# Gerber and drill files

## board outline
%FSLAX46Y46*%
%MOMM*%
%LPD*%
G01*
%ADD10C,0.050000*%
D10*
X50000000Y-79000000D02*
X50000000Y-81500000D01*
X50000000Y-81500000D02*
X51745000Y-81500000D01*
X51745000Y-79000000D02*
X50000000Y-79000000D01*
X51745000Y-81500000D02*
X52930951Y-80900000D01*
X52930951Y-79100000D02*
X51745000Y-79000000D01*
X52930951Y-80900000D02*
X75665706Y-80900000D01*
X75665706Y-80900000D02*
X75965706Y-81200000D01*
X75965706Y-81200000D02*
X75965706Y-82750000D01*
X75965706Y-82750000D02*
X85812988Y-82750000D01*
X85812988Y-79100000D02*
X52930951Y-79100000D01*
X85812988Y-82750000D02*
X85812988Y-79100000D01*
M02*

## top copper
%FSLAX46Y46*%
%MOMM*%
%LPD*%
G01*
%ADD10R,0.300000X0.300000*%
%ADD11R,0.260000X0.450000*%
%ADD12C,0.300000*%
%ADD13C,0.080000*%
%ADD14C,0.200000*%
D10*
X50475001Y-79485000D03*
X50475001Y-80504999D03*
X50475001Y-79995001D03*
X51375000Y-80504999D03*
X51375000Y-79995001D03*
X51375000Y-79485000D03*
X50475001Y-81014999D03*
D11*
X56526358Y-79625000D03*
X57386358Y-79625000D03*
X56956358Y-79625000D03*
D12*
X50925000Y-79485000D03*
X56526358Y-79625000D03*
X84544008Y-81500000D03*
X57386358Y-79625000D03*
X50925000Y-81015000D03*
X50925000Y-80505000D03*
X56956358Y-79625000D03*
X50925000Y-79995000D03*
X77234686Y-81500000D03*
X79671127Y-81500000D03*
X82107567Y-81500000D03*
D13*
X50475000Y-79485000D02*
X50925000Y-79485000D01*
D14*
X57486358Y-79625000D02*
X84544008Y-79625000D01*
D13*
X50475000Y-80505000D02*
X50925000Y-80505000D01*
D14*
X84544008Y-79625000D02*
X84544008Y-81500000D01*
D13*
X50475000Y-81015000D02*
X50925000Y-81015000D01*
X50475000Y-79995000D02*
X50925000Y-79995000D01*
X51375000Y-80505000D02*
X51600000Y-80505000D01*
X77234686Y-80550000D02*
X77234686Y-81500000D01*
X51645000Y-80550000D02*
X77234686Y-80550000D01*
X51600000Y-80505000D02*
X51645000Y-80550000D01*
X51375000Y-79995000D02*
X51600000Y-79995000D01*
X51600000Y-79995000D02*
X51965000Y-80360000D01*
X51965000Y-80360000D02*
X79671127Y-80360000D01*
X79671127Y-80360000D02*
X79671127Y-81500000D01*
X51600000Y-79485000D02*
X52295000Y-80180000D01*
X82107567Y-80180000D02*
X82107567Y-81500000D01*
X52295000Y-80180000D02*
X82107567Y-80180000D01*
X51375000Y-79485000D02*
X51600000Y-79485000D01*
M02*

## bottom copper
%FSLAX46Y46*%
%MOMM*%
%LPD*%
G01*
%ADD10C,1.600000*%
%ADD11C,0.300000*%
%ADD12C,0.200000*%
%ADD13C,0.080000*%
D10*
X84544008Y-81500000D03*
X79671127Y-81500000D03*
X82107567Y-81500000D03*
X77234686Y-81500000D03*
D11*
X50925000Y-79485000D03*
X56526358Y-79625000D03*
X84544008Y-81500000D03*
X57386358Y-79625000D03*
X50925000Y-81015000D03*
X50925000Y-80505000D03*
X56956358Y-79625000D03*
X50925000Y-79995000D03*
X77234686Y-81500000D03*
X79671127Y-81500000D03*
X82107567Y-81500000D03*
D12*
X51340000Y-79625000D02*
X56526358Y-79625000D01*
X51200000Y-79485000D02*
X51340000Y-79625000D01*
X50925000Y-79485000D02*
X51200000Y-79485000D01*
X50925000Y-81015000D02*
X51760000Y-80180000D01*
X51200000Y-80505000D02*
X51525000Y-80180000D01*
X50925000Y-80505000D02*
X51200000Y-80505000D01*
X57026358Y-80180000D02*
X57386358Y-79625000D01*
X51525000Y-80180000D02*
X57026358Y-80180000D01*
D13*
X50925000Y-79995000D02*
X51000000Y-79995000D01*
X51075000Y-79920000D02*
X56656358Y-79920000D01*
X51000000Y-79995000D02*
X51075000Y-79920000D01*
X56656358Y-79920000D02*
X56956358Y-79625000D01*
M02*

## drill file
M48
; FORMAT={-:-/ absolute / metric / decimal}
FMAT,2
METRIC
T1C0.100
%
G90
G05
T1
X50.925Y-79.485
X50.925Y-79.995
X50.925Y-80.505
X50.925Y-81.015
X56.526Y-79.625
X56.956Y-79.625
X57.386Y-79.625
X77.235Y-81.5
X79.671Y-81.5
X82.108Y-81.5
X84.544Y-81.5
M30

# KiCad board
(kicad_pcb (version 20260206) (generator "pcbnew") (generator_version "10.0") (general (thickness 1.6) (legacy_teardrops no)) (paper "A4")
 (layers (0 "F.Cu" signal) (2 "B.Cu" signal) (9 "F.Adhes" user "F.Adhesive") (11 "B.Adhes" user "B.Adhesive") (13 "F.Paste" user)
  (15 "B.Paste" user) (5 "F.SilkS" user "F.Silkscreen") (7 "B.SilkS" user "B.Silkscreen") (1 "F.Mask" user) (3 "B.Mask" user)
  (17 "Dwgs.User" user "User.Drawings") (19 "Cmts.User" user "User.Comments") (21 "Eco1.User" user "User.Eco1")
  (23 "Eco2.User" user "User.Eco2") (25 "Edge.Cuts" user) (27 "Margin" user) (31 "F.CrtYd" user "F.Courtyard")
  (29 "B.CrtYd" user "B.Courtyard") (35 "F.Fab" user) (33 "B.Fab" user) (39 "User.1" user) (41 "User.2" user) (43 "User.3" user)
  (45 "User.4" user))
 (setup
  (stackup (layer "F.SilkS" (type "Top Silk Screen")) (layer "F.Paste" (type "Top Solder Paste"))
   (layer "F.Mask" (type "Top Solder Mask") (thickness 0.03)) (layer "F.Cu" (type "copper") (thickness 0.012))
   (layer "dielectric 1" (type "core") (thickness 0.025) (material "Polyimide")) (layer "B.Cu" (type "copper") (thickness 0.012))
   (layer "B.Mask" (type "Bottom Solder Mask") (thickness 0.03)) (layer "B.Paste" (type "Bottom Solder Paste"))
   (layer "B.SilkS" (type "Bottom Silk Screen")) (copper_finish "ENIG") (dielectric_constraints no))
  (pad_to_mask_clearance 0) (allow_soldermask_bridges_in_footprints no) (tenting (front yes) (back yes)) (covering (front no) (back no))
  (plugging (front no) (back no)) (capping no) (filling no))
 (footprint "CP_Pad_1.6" (layer "F.Cu") (at 84.544008 81.5)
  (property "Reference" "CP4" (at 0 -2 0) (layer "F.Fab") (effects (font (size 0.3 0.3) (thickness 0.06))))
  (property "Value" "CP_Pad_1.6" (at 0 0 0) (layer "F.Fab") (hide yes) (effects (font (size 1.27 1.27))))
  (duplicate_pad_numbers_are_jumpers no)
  (pad "1" smd circle (at 0 0) (size 1.6 1.6) (layers "B.Cu" "B.Mask") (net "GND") (solder_mask_margin 0.1)))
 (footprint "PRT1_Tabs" (layer "F.Cu") (at 56.956358 79.625)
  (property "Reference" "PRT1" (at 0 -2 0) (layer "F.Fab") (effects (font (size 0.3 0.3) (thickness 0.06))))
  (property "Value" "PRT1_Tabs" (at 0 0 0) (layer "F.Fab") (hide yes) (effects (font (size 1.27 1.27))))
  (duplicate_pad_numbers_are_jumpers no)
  (pad "1" smd rect (at -0.43 0) (size 0.26 0.45) (layers "F.Cu" "F.Mask") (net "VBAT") (solder_mask_margin 0.05) (thermal_bridge_angle 45))
  (pad "2" smd rect (at 0.43 0) (size 0.26 0.45) (layers "F.Cu" "F.Mask") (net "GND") (solder_mask_margin 0.05) (thermal_bridge_angle 45))
  (pad "3" smd rect (at 0 0) (size 0.26 0.45) (layers "F.Cu" "F.Mask") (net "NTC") (solder_mask_margin 0.05) (thermal_bridge_angle 45)))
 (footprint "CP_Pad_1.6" (layer "F.Cu") (at 77.234686 81.5)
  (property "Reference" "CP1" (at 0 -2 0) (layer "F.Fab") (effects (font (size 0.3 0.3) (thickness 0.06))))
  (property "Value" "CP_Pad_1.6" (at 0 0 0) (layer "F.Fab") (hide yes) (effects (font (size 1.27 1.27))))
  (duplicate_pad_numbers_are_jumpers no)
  (pad "1" smd circle (at 0 0) (size 1.6 1.6) (layers "B.Cu" "B.Mask") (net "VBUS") (solder_mask_margin 0.1)))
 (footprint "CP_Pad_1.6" (layer "F.Cu") (at 79.671127 81.5)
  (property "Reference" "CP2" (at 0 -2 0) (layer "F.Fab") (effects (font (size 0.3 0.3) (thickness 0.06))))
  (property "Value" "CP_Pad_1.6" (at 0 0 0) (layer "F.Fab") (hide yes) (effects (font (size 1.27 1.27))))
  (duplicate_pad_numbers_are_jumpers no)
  (pad "1" smd circle (at 0 0) (size 1.6 1.6) (layers "B.Cu" "B.Mask") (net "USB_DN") (solder_mask_margin 0.1)))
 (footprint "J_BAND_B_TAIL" (layer "F.Cu") (at 50.9 80.25)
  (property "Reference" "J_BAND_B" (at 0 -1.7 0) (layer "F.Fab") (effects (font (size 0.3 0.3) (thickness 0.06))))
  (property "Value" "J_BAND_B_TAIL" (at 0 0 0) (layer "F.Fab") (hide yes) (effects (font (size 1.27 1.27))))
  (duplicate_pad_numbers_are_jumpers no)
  (pad "1" smd rect (at -0.424999 -0.765) (size 0.3 0.3) (layers "F.Cu" "F.Mask") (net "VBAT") (solder_mask_margin 0.05)
   (thermal_bridge_angle 45))
  (pad "2" smd rect (at -0.424999 0.254999) (size 0.3 0.3) (layers "F.Cu" "F.Mask") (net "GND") (solder_mask_margin 0.05)
   (thermal_bridge_angle 45))
  (pad "3" smd rect (at -0.424999 -0.254999) (size 0.3 0.3) (layers "F.Cu" "F.Mask") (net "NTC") (solder_mask_margin 0.05)
   (thermal_bridge_angle 45))
  (pad "4" smd rect (at 0.475 0.254999) (size 0.3 0.3) (layers "F.Cu" "F.Mask") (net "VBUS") (solder_mask_margin 0.05)
   (thermal_bridge_angle 45))
  (pad "5" smd rect (at 0.475 -0.254999) (size 0.3 0.3) (layers "F.Cu" "F.Mask") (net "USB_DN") (solder_mask_margin 0.05)
   (thermal_bridge_angle 45))
  (pad "6" smd rect (at 0.475 -0.765) (size 0.3 0.3) (layers "F.Cu" "F.Mask") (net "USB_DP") (solder_mask_margin 0.05)
   (thermal_bridge_angle 45))
  (pad "7" smd rect (at -0.424999 0.764999) (size 0.3 0.3) (layers "F.Cu" "F.Mask") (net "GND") (solder_mask_margin 0.05)
   (thermal_bridge_angle 45)))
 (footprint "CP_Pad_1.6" (layer "F.Cu") (at 82.107567 81.5)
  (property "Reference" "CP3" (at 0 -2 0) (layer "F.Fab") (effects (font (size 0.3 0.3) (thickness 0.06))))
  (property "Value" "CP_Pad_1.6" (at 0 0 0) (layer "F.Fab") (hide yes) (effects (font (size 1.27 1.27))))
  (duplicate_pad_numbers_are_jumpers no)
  (pad "1" smd circle (at 0 0) (size 1.6 1.6) (layers "B.Cu" "B.Mask") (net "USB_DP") (solder_mask_margin 0.1)))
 (gr_line (start 50 79) (end 50 81.5) (stroke (width 0.05) (type default)) (layer "Edge.Cuts"))
 (gr_line (start 50 81.5) (end 51.745 81.5) (stroke (width 0.05) (type default)) (layer "Edge.Cuts"))
 (gr_line (start 51.745 79) (end 50 79) (stroke (width 0.05) (type default)) (layer "Edge.Cuts"))
 (gr_line (start 51.745 81.5) (end 52.930951 80.9) (stroke (width 0.05) (type default)) (layer "Edge.Cuts"))
 (gr_line (start 52.930951 79.1) (end 51.745 79) (stroke (width 0.05) (type default)) (layer "Edge.Cuts"))
 (gr_line (start 52.930951 80.9) (end 75.665706 80.9) (stroke (width 0.05) (type default)) (layer "Edge.Cuts"))
 (gr_line (start 75.665706 80.9) (end 75.965706 81.2) (stroke (width 0.05) (type default)) (layer "Edge.Cuts"))
 (gr_line (start 75.965706 81.2) (end 75.965706 82.75) (stroke (width 0.05) (type default)) (layer "Edge.Cuts"))
 (gr_line (start 75.965706 82.75) (end 85.812988 82.75) (stroke (width 0.05) (type default)) (layer "Edge.Cuts"))
 (gr_line (start 85.812988 79.1) (end 52.930951 79.1) (stroke (width 0.05) (type default)) (layer "Edge.Cuts"))
 (gr_line (start 85.812988 82.75) (end 85.812988 79.1) (stroke (width 0.05) (type default)) (layer "Edge.Cuts"))
 (segment (start 50.475 79.485) (end 50.925 79.485) (width 0.08) (layer "F.Cu") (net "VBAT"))
 (via (at 56.526358 79.625) (size 0.3) (drill 0.1) (layers "F.Cu" "B.Cu") (tenting (front yes) (back yes)) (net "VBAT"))
 (via (at 50.925 79.485) (size 0.3) (drill 0.1) (layers "F.Cu" "B.Cu") (tenting (front yes) (back yes)) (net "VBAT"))
 (segment (start 50.925 79.485) (end 51.2 79.485) (width 0.2) (layer "B.Cu") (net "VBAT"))
 (segment (start 51.2 79.485) (end 51.34 79.625) (width 0.2) (layer "B.Cu") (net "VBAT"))
 (segment (start 51.34 79.625) (end 56.526358 79.625) (width 0.2) (layer "B.Cu") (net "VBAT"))
 (segment (start 50.475 80.505) (end 50.925 80.505) (width 0.08) (layer "F.Cu") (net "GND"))
 (segment (start 57.486358 79.625) (end 84.544008 79.625) (width 0.2) (layer "F.Cu") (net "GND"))
 (segment (start 50.475 81.015) (end 50.925 81.015) (width 0.08) (layer "F.Cu") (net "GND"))
 (segment (start 84.544008 79.625) (end 84.544008 81.5) (width 0.2) (layer "F.Cu") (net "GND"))
 (via (at 50.925 80.505) (size 0.3) (drill 0.1) (layers "F.Cu" "B.Cu") (tenting (front yes) (back yes)) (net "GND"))
 (via (at 84.544008 81.5) (size 0.3) (drill 0.1) (layers "F.Cu" "B.Cu") (tenting (front yes) (back yes)) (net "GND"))
 (via (at 57.386358 79.625) (size 0.3) (drill 0.1) (layers "F.Cu" "B.Cu") (tenting (front yes) (back yes)) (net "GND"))
 (via (at 50.925 81.015) (size 0.3) (drill 0.1) (layers "F.Cu" "B.Cu") (tenting (front yes) (back yes)) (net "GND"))
 (segment (start 50.925 80.505) (end 51.2 80.505) (width 0.2) (layer "B.Cu") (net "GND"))
 (segment (start 57.026358 80.18) (end 57.386358 79.625) (width 0.2) (layer "B.Cu") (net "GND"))
 (segment (start 51.2 80.505) (end 51.525 80.18) (width 0.2) (layer "B.Cu") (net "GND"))
 (segment (start 51.525 80.18) (end 57.026358 80.18) (width 0.2) (layer "B.Cu") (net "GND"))
 (segment (start 50.925 81.015) (end 51.76 80.18) (width 0.2) (layer "B.Cu") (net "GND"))
 (segment (start 50.475 79.995) (end 50.925 79.995) (width 0.08) (layer "F.Cu") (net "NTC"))
 (via (at 50.925 79.995) (size 0.3) (drill 0.1) (layers "F.Cu" "B.Cu") (tenting (front yes) (back yes)) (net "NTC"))
 (via (at 56.956358 79.625) (size 0.3) (drill 0.1) (layers "F.Cu" "B.Cu") (tenting (front yes) (back yes)) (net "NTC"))
 (segment (start 51.075 79.92) (end 56.656358 79.92) (width 0.08) (layer "B.Cu") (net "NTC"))
 (segment (start 51 79.995) (end 51.075 79.92) (width 0.08) (layer "B.Cu") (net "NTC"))
 (segment (start 50.925 79.995) (end 51 79.995) (width 0.08) (layer "B.Cu") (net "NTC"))
 (segment (start 56.656358 79.92) (end 56.956358 79.625) (width 0.08) (layer "B.Cu") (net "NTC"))
 (segment (start 77.234686 80.55) (end 77.234686 81.5) (width 0.08) (layer "F.Cu") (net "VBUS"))
 (segment (start 51.375 80.505) (end 51.6 80.505) (width 0.08) (layer "F.Cu") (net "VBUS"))
 (segment (start 51.6 80.505) (end 51.645 80.55) (width 0.08) (layer "F.Cu") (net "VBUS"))
 (segment (start 51.645 80.55) (end 77.234686 80.55) (width 0.08) (layer "F.Cu") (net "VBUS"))
 (via (at 77.234686 81.5) (size 0.3) (drill 0.1) (layers "F.Cu" "B.Cu") (tenting (front yes) (back yes)) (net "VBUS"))
 (segment (start 51.965 80.36) (end 79.671127 80.36) (width 0.08) (layer "F.Cu") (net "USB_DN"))
 (segment (start 51.375 79.995) (end 51.6 79.995) (width 0.08) (layer "F.Cu") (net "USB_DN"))
 (segment (start 51.6 79.995) (end 51.965 80.36) (width 0.08) (layer "F.Cu") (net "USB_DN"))
 (segment (start 79.671127 80.36) (end 79.671127 81.5) (width 0.08) (layer "F.Cu") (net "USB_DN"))
 (via (at 79.671127 81.5) (size 0.3) (drill 0.1) (layers "F.Cu" "B.Cu") (tenting (front yes) (back yes)) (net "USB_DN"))
 (segment (start 52.295 80.18) (end 82.107567 80.18) (width 0.08) (layer "F.Cu") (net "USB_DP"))
 (segment (start 51.375 79.485) (end 51.6 79.485) (width 0.08) (layer "F.Cu") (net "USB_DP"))
 (segment (start 82.107567 80.18) (end 82.107567 81.5) (width 0.08) (layer "F.Cu") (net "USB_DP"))
 (segment (start 51.6 79.485) (end 52.295 80.18) (width 0.08) (layer "F.Cu") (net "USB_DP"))
 (via (at 82.107567 81.5) (size 0.3) (drill 0.1) (layers "F.Cu" "B.Cu") (tenting (front yes) (back yes)) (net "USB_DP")))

